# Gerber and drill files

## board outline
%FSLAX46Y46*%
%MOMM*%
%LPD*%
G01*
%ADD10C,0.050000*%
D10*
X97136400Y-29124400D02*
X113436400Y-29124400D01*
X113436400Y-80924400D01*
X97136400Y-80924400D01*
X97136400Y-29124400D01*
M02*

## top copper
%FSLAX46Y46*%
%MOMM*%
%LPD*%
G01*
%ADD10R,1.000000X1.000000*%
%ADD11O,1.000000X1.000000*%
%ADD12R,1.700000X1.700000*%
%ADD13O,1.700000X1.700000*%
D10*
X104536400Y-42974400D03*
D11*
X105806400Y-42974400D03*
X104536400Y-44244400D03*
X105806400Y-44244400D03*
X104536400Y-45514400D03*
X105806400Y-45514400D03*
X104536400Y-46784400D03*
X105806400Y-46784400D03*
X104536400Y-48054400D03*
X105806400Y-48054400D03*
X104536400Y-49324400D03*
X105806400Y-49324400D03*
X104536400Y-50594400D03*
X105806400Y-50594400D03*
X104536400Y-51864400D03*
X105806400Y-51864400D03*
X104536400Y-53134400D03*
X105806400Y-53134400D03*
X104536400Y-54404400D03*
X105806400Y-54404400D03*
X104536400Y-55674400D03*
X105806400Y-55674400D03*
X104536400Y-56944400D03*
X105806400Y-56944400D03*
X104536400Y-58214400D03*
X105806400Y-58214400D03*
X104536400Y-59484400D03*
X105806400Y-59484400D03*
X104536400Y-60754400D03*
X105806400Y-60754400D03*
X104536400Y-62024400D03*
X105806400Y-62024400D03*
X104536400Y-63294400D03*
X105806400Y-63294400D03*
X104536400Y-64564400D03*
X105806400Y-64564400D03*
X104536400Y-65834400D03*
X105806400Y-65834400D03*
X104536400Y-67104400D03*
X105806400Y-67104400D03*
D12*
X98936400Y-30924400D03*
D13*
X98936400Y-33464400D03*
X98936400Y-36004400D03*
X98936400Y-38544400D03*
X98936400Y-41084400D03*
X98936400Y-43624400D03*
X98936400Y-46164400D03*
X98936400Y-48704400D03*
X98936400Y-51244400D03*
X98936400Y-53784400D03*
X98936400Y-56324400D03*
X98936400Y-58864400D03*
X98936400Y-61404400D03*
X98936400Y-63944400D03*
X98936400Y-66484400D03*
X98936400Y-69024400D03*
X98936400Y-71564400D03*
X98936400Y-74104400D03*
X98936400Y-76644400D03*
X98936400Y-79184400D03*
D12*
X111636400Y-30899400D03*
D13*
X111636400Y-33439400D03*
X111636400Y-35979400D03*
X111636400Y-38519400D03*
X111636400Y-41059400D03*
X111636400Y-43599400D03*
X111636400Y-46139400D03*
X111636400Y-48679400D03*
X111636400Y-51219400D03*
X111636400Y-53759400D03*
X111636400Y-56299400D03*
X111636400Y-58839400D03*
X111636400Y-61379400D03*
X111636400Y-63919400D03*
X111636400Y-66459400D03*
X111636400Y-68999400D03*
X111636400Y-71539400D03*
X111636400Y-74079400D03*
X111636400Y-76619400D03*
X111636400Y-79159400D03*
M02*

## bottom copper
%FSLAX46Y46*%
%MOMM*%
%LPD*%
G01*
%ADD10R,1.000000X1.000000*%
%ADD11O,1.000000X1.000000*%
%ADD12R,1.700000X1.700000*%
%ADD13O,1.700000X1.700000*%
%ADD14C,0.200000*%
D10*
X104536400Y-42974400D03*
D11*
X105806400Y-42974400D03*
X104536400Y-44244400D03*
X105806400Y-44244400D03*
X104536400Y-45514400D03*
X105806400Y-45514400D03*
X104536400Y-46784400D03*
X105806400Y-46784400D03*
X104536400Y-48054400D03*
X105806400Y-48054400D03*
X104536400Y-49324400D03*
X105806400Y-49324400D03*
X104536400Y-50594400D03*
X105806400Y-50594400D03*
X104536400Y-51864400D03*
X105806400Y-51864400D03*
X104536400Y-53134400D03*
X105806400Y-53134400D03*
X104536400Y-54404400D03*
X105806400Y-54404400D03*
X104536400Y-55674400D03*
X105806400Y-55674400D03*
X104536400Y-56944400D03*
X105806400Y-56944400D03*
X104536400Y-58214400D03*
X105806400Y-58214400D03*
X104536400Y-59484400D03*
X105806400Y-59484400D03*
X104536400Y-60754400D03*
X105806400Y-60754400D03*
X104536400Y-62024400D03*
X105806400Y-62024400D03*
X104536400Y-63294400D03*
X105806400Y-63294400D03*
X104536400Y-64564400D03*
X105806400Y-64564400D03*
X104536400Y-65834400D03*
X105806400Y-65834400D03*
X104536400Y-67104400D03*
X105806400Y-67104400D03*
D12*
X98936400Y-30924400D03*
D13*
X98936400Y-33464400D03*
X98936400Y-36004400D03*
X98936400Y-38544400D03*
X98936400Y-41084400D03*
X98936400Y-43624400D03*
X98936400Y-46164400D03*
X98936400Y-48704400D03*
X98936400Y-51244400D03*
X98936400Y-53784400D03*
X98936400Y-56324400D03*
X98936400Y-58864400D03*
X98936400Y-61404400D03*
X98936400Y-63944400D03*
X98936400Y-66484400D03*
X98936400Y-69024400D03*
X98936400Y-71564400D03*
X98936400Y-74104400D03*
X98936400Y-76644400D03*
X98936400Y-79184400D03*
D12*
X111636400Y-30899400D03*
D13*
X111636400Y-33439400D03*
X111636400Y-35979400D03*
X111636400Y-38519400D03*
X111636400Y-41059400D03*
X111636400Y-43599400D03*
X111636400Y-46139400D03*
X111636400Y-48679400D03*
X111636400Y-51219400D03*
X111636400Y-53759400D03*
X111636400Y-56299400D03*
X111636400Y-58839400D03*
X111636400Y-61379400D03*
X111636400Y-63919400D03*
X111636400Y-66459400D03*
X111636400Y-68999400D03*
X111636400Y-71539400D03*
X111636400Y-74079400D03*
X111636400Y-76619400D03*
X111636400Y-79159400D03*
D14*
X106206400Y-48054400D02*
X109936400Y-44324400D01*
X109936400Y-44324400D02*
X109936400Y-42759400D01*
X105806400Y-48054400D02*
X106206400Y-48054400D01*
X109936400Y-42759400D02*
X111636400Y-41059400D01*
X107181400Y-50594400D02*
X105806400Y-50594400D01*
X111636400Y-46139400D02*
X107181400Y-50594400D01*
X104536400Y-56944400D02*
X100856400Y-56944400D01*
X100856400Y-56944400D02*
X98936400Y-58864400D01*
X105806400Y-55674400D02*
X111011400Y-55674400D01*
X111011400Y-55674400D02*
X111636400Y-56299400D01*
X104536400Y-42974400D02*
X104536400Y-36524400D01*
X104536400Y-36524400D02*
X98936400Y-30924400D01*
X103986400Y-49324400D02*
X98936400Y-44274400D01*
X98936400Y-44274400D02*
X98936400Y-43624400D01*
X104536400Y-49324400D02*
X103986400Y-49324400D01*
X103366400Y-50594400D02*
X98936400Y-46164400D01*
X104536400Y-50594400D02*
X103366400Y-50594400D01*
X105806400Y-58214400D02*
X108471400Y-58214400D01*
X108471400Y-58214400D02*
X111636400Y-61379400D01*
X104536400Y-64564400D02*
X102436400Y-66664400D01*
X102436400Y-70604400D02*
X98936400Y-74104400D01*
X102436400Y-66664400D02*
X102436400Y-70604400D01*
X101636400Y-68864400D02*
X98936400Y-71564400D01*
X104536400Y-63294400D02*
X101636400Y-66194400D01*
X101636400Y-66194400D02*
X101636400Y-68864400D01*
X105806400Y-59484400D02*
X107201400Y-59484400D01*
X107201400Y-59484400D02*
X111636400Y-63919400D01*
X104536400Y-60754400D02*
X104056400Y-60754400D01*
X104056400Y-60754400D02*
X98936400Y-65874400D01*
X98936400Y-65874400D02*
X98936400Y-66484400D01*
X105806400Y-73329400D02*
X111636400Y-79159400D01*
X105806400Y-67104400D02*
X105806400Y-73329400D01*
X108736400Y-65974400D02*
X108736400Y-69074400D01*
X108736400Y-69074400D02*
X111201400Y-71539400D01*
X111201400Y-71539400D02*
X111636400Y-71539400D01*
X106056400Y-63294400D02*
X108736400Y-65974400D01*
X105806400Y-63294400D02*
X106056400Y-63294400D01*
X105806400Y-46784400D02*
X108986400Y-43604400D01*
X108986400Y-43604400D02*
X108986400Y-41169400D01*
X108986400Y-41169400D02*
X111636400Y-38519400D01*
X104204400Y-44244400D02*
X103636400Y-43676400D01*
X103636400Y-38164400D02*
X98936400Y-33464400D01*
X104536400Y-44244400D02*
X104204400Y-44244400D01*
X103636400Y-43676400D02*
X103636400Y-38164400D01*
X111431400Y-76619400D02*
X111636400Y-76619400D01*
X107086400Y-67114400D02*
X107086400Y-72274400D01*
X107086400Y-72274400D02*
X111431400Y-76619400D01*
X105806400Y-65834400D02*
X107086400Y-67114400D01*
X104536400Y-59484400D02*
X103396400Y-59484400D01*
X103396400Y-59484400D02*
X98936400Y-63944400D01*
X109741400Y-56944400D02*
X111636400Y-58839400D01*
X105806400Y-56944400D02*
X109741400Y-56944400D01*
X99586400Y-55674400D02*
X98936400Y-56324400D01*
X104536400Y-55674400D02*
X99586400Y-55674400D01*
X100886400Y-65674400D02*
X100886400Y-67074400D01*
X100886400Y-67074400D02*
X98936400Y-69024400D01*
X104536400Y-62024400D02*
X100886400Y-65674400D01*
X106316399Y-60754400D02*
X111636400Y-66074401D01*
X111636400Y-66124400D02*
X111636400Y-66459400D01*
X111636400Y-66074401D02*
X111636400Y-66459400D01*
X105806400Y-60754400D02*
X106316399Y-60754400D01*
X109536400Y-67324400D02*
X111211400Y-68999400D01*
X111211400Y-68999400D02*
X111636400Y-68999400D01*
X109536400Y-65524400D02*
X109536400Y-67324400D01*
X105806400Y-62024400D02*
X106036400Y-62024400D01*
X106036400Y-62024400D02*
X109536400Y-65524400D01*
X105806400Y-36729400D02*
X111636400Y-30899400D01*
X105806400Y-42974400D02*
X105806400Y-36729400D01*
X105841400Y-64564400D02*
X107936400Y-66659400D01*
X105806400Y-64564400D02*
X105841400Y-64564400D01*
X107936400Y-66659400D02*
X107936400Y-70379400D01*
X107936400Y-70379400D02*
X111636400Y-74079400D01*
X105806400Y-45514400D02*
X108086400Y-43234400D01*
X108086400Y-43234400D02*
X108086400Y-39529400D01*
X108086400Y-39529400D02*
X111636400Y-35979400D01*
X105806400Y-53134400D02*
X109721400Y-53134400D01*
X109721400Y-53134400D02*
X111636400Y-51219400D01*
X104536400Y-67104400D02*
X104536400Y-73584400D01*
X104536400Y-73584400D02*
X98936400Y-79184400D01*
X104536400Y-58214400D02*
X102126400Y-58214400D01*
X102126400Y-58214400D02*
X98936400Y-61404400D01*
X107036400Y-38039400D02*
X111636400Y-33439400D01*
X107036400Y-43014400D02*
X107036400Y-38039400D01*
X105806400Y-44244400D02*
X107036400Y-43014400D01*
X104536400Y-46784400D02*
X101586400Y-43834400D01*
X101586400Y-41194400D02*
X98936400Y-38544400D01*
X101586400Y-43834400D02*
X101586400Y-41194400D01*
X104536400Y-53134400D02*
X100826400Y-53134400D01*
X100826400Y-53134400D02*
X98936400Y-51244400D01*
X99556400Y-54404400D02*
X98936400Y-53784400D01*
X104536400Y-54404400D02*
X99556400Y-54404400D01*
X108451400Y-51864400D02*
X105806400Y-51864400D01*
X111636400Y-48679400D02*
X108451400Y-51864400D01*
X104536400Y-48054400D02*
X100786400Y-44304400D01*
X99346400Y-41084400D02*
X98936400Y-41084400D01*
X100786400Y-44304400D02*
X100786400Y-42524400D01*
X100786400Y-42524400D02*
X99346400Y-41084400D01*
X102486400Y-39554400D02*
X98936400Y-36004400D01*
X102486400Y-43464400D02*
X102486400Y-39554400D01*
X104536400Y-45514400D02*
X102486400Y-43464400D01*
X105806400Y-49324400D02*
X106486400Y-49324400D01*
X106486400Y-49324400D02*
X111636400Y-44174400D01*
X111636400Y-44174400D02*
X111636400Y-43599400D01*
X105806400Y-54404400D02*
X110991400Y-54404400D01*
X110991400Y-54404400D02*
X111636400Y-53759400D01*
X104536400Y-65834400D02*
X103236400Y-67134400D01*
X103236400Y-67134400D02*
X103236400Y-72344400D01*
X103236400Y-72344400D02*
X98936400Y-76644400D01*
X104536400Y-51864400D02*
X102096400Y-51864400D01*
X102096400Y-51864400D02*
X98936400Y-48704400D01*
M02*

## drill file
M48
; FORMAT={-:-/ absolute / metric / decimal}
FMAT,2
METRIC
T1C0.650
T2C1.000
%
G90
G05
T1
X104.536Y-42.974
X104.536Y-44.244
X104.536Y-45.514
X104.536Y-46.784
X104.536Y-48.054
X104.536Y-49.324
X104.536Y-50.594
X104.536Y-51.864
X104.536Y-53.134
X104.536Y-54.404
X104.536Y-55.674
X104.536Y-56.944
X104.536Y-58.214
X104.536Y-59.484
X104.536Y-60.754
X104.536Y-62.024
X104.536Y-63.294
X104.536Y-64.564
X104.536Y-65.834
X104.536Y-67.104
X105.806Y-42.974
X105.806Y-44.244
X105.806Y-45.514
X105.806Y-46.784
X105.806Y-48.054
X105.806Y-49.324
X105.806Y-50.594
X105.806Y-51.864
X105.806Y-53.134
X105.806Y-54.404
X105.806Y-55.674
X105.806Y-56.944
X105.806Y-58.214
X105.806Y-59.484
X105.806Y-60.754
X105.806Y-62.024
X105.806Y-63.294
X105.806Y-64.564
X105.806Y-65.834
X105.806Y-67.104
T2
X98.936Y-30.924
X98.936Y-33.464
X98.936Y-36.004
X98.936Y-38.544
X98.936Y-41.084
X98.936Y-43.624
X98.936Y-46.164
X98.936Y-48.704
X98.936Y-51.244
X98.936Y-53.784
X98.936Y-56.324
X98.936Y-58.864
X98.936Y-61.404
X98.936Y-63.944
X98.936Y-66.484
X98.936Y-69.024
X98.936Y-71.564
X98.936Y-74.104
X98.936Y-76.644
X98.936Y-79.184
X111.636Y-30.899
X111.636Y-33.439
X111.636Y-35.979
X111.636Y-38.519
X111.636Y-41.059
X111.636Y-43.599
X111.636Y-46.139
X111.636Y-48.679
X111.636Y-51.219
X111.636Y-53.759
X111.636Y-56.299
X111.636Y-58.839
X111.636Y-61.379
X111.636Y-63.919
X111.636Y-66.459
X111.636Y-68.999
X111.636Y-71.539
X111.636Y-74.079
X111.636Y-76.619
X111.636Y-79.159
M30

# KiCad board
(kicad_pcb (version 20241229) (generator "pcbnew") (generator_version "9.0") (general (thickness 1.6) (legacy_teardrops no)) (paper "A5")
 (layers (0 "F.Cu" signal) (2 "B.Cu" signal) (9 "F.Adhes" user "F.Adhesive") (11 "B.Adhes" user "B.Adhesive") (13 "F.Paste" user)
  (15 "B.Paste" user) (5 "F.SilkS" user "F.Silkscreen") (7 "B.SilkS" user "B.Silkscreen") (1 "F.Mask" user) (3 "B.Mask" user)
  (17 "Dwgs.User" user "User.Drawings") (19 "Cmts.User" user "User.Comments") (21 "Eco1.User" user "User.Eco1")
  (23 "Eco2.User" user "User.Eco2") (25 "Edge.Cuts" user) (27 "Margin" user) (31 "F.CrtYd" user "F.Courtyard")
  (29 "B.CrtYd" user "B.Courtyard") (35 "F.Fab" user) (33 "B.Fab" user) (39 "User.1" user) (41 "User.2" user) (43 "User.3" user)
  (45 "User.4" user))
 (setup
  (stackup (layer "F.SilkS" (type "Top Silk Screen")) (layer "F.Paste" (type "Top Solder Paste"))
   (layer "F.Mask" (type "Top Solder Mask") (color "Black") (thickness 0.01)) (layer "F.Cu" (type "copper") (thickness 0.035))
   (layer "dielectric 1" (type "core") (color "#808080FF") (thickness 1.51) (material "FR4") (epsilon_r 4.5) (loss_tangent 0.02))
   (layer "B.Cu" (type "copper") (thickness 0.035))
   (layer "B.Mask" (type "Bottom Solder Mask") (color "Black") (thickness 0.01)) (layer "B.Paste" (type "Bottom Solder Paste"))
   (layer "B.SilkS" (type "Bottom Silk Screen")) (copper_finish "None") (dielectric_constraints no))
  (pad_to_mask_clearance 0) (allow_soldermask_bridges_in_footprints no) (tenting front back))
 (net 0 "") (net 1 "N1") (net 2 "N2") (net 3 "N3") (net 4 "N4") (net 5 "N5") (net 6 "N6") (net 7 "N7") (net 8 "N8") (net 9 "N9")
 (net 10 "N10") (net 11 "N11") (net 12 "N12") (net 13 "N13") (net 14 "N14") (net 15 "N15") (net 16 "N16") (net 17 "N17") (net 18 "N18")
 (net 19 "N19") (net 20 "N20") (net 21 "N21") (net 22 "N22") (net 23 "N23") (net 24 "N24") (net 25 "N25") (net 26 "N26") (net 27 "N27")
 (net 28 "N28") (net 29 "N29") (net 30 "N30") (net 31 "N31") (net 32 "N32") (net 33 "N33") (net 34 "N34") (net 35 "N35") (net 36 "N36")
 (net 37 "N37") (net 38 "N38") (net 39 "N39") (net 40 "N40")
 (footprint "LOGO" (layer "F.Cu") (at 105.3988 74.55 90)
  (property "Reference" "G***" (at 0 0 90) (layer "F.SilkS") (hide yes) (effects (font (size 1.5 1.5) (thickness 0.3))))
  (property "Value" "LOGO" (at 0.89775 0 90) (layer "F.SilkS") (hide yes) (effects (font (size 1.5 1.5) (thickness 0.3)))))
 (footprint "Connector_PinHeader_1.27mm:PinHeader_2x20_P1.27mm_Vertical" (layer "F.Cu") (at 104.5364 42.9744)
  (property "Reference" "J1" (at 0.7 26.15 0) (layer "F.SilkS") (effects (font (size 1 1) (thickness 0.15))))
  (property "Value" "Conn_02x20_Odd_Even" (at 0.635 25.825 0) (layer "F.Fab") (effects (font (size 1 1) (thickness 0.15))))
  (pad "1" thru_hole rect (at 0 0) (size 1 1) (drill 0.65) (layers "*.Cu" "*.Mask") (remove_unused_layers no) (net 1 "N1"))
  (pad "2" thru_hole oval (at 1.27 0) (size 1 1) (drill 0.65) (layers "*.Cu" "*.Mask") (remove_unused_layers no) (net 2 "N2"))
  (pad "3" thru_hole oval (at 0 1.27) (size 1 1) (drill 0.65) (layers "*.Cu" "*.Mask") (remove_unused_layers no) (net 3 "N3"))
  (pad "4" thru_hole oval (at 1.27 1.27) (size 1 1) (drill 0.65) (layers "*.Cu" "*.Mask") (remove_unused_layers no) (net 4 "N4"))
  (pad "5" thru_hole oval (at 0 2.54) (size 1 1) (drill 0.65) (layers "*.Cu" "*.Mask") (remove_unused_layers no) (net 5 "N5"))
  (pad "6" thru_hole oval (at 1.27 2.54) (size 1 1) (drill 0.65) (layers "*.Cu" "*.Mask") (remove_unused_layers no) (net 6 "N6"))
  (pad "7" thru_hole oval (at 0 3.81) (size 1 1) (drill 0.65) (layers "*.Cu" "*.Mask") (remove_unused_layers no) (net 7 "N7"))
  (pad "8" thru_hole oval (at 1.27 3.81) (size 1 1) (drill 0.65) (layers "*.Cu" "*.Mask") (remove_unused_layers no) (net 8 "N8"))
  (pad "9" thru_hole oval (at 0 5.08) (size 1 1) (drill 0.65) (layers "*.Cu" "*.Mask") (remove_unused_layers no) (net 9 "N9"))
  (pad "10" thru_hole oval (at 1.27 5.08) (size 1 1) (drill 0.65) (layers "*.Cu" "*.Mask") (remove_unused_layers no) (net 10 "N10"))
  (pad "11" thru_hole oval (at 0 6.35) (size 1 1) (drill 0.65) (layers "*.Cu" "*.Mask") (remove_unused_layers no) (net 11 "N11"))
  (pad "12" thru_hole oval (at 1.27 6.35) (size 1 1) (drill 0.65) (layers "*.Cu" "*.Mask") (remove_unused_layers no) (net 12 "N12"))
  (pad "13" thru_hole oval (at 0 7.62) (size 1 1) (drill 0.65) (layers "*.Cu" "*.Mask") (remove_unused_layers no) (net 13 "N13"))
  (pad "14" thru_hole oval (at 1.27 7.62) (size 1 1) (drill 0.65) (layers "*.Cu" "*.Mask") (remove_unused_layers no) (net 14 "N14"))
  (pad "15" thru_hole oval (at 0 8.89) (size 1 1) (drill 0.65) (layers "*.Cu" "*.Mask") (remove_unused_layers no) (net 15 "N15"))
  (pad "16" thru_hole oval (at 1.27 8.89) (size 1 1) (drill 0.65) (layers "*.Cu" "*.Mask") (remove_unused_layers no) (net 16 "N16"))
  (pad "17" thru_hole oval (at 0 10.16) (size 1 1) (drill 0.65) (layers "*.Cu" "*.Mask") (remove_unused_layers no) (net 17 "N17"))
  (pad "18" thru_hole oval (at 1.27 10.16) (size 1 1) (drill 0.65) (layers "*.Cu" "*.Mask") (remove_unused_layers no) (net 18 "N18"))
  (pad "19" thru_hole oval (at 0 11.43) (size 1 1) (drill 0.65) (layers "*.Cu" "*.Mask") (remove_unused_layers no) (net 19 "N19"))
  (pad "20" thru_hole oval (at 1.27 11.43) (size 1 1) (drill 0.65) (layers "*.Cu" "*.Mask") (remove_unused_layers no) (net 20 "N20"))
  (pad "21" thru_hole oval (at 0 12.7) (size 1 1) (drill 0.65) (layers "*.Cu" "*.Mask") (remove_unused_layers no) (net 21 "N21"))
  (pad "22" thru_hole oval (at 1.27 12.7) (size 1 1) (drill 0.65) (layers "*.Cu" "*.Mask") (remove_unused_layers no) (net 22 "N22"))
  (pad "23" thru_hole oval (at 0 13.97) (size 1 1) (drill 0.65) (layers "*.Cu" "*.Mask") (remove_unused_layers no) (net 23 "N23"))
  (pad "24" thru_hole oval (at 1.27 13.97) (size 1 1) (drill 0.65) (layers "*.Cu" "*.Mask") (remove_unused_layers no) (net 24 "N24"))
  (pad "25" thru_hole oval (at 0 15.24) (size 1 1) (drill 0.65) (layers "*.Cu" "*.Mask") (remove_unused_layers no) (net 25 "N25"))
  (pad "26" thru_hole oval (at 1.27 15.24) (size 1 1) (drill 0.65) (layers "*.Cu" "*.Mask") (remove_unused_layers no) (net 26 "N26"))
  (pad "27" thru_hole oval (at 0 16.51) (size 1 1) (drill 0.65) (layers "*.Cu" "*.Mask") (remove_unused_layers no) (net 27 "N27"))
  (pad "28" thru_hole oval (at 1.27 16.51) (size 1 1) (drill 0.65) (layers "*.Cu" "*.Mask") (remove_unused_layers no) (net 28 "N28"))
  (pad "29" thru_hole oval (at 0 17.78) (size 1 1) (drill 0.65) (layers "*.Cu" "*.Mask") (remove_unused_layers no) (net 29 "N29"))
  (pad "30" thru_hole oval (at 1.27 17.78) (size 1 1) (drill 0.65) (layers "*.Cu" "*.Mask") (remove_unused_layers no) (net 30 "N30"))
  (pad "31" thru_hole oval (at 0 19.05) (size 1 1) (drill 0.65) (layers "*.Cu" "*.Mask") (remove_unused_layers no) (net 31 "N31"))
  (pad "32" thru_hole oval (at 1.27 19.05) (size 1 1) (drill 0.65) (layers "*.Cu" "*.Mask") (remove_unused_layers no) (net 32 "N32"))
  (pad "33" thru_hole oval (at 0 20.32) (size 1 1) (drill 0.65) (layers "*.Cu" "*.Mask") (remove_unused_layers no) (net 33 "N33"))
  (pad "34" thru_hole oval (at 1.27 20.32) (size 1 1) (drill 0.65) (layers "*.Cu" "*.Mask") (remove_unused_layers no) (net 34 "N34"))
  (pad "35" thru_hole oval (at 0 21.59) (size 1 1) (drill 0.65) (layers "*.Cu" "*.Mask") (remove_unused_layers no) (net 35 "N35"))
  (pad "36" thru_hole oval (at 1.27 21.59) (size 1 1) (drill 0.65) (layers "*.Cu" "*.Mask") (remove_unused_layers no) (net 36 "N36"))
  (pad "37" thru_hole oval (at 0 22.86) (size 1 1) (drill 0.65) (layers "*.Cu" "*.Mask") (remove_unused_layers no) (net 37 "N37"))
  (pad "38" thru_hole oval (at 1.27 22.86) (size 1 1) (drill 0.65) (layers "*.Cu" "*.Mask") (remove_unused_layers no) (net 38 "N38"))
  (pad "39" thru_hole oval (at 0 24.13) (size 1 1) (drill 0.65) (layers "*.Cu" "*.Mask") (remove_unused_layers no) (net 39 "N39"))
  (pad "40" thru_hole oval (at 1.27 24.13) (size 1 1) (drill 0.65) (layers "*.Cu" "*.Mask") (remove_unused_layers no) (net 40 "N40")))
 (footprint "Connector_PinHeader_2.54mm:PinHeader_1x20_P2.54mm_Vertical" (layer "B.Cu") (at 98.9364 30.9244 180)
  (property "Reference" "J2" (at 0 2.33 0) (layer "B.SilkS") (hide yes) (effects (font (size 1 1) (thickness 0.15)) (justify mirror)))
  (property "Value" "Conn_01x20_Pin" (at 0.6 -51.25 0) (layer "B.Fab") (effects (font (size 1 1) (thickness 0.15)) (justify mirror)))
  (pad "1" thru_hole rect (at 0 0 180) (size 1.7 1.7) (drill 1) (layers "*.Cu" "*.Mask") (remove_unused_layers no) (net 1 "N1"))
  (pad "2" thru_hole oval (at 0 -2.54 180) (size 1.7 1.7) (drill 1) (layers "*.Cu" "*.Mask") (remove_unused_layers no) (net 3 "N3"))
  (pad "3" thru_hole oval (at 0 -5.08 180) (size 1.7 1.7) (drill 1) (layers "*.Cu" "*.Mask") (remove_unused_layers no) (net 5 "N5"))
  (pad "4" thru_hole oval (at 0 -7.62 180) (size 1.7 1.7) (drill 1) (layers "*.Cu" "*.Mask") (remove_unused_layers no) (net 7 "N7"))
  (pad "5" thru_hole oval (at 0 -10.16 180) (size 1.7 1.7) (drill 1) (layers "*.Cu" "*.Mask") (remove_unused_layers no) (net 9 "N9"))
  (pad "6" thru_hole oval (at 0 -12.7 180) (size 1.7 1.7) (drill 1) (layers "*.Cu" "*.Mask") (remove_unused_layers no) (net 11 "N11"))
  (pad "7" thru_hole oval (at 0 -15.24 180) (size 1.7 1.7) (drill 1) (layers "*.Cu" "*.Mask") (remove_unused_layers no) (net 13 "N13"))
  (pad "8" thru_hole oval (at 0 -17.78 180) (size 1.7 1.7) (drill 1) (layers "*.Cu" "*.Mask") (remove_unused_layers no) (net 15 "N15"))
  (pad "9" thru_hole oval (at 0 -20.32 180) (size 1.7 1.7) (drill 1) (layers "*.Cu" "*.Mask") (remove_unused_layers no) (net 17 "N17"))
  (pad "10" thru_hole oval (at 0 -22.86 180) (size 1.7 1.7) (drill 1) (layers "*.Cu" "*.Mask") (remove_unused_layers no) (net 19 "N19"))
  (pad "11" thru_hole oval (at 0 -25.4 180) (size 1.7 1.7) (drill 1) (layers "*.Cu" "*.Mask") (remove_unused_layers no) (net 21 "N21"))
  (pad "12" thru_hole oval (at 0 -27.94 180) (size 1.7 1.7) (drill 1) (layers "*.Cu" "*.Mask") (remove_unused_layers no) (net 23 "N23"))
  (pad "13" thru_hole oval (at 0 -30.48 180) (size 1.7 1.7) (drill 1) (layers "*.Cu" "*.Mask") (remove_unused_layers no) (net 25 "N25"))
  (pad "14" thru_hole oval (at 0 -33.02 180) (size 1.7 1.7) (drill 1) (layers "*.Cu" "*.Mask") (remove_unused_layers no) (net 27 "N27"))
  (pad "15" thru_hole oval (at 0 -35.56 180) (size 1.7 1.7) (drill 1) (layers "*.Cu" "*.Mask") (remove_unused_layers no) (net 29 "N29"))
  (pad "16" thru_hole oval (at 0 -38.1 180) (size 1.7 1.7) (drill 1) (layers "*.Cu" "*.Mask") (remove_unused_layers no) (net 31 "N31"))
  (pad "17" thru_hole oval (at 0 -40.64 180) (size 1.7 1.7) (drill 1) (layers "*.Cu" "*.Mask") (remove_unused_layers no) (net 33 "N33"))
  (pad "18" thru_hole oval (at 0 -43.18 180) (size 1.7 1.7) (drill 1) (layers "*.Cu" "*.Mask") (remove_unused_layers no) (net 35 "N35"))
  (pad "19" thru_hole oval (at 0 -45.72 180) (size 1.7 1.7) (drill 1) (layers "*.Cu" "*.Mask") (remove_unused_layers no) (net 37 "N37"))
  (pad "20" thru_hole oval (at 0 -48.26 180) (size 1.7 1.7) (drill 1) (layers "*.Cu" "*.Mask") (remove_unused_layers no) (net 39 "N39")))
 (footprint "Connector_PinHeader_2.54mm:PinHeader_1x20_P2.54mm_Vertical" (layer "B.Cu") (at 111.6364 30.8994 180)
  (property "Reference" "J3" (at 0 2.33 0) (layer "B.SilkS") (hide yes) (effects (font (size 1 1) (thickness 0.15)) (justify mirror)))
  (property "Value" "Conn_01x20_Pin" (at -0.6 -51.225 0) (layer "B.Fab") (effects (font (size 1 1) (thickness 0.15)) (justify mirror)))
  (pad "1" thru_hole rect (at 0 0 180) (size 1.7 1.7) (drill 1) (layers "*.Cu" "*.Mask") (remove_unused_layers no) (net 2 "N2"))
  (pad "2" thru_hole oval (at 0 -2.54 180) (size 1.7 1.7) (drill 1) (layers "*.Cu" "*.Mask") (remove_unused_layers no) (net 4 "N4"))
  (pad "3" thru_hole oval (at 0 -5.08 180) (size 1.7 1.7) (drill 1) (layers "*.Cu" "*.Mask") (remove_unused_layers no) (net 6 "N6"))
  (pad "4" thru_hole oval (at 0 -7.62 180) (size 1.7 1.7) (drill 1) (layers "*.Cu" "*.Mask") (remove_unused_layers no) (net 8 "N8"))
  (pad "5" thru_hole oval (at 0 -10.16 180) (size 1.7 1.7) (drill 1) (layers "*.Cu" "*.Mask") (remove_unused_layers no) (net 10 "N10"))
  (pad "6" thru_hole oval (at 0 -12.7 180) (size 1.7 1.7) (drill 1) (layers "*.Cu" "*.Mask") (remove_unused_layers no) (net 12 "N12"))
  (pad "7" thru_hole oval (at 0 -15.24 180) (size 1.7 1.7) (drill 1) (layers "*.Cu" "*.Mask") (remove_unused_layers no) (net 14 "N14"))
  (pad "8" thru_hole oval (at 0 -17.78 180) (size 1.7 1.7) (drill 1) (layers "*.Cu" "*.Mask") (remove_unused_layers no) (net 16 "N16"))
  (pad "9" thru_hole oval (at 0 -20.32 180) (size 1.7 1.7) (drill 1) (layers "*.Cu" "*.Mask") (remove_unused_layers no) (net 18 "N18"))
  (pad "10" thru_hole oval (at 0 -22.86 180) (size 1.7 1.7) (drill 1) (layers "*.Cu" "*.Mask") (remove_unused_layers no) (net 20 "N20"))
  (pad "11" thru_hole oval (at 0 -25.4 180) (size 1.7 1.7) (drill 1) (layers "*.Cu" "*.Mask") (remove_unused_layers no) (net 22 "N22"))
  (pad "12" thru_hole oval (at 0 -27.94 180) (size 1.7 1.7) (drill 1) (layers "*.Cu" "*.Mask") (remove_unused_layers no) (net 24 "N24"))
  (pad "13" thru_hole oval (at 0 -30.48 180) (size 1.7 1.7) (drill 1) (layers "*.Cu" "*.Mask") (remove_unused_layers no) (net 26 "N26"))
  (pad "14" thru_hole oval (at 0 -33.02 180) (size 1.7 1.7) (drill 1) (layers "*.Cu" "*.Mask") (remove_unused_layers no) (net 28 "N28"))
  (pad "15" thru_hole oval (at 0 -35.56 180) (size 1.7 1.7) (drill 1) (layers "*.Cu" "*.Mask") (remove_unused_layers no) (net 30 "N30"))
  (pad "16" thru_hole oval (at 0 -38.1 180) (size 1.7 1.7) (drill 1) (layers "*.Cu" "*.Mask") (remove_unused_layers no) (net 32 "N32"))
  (pad "17" thru_hole oval (at 0 -40.64 180) (size 1.7 1.7) (drill 1) (layers "*.Cu" "*.Mask") (remove_unused_layers no) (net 34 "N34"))
  (pad "18" thru_hole oval (at 0 -43.18 180) (size 1.7 1.7) (drill 1) (layers "*.Cu" "*.Mask") (remove_unused_layers no) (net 36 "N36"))
  (pad "19" thru_hole oval (at 0 -45.72 180) (size 1.7 1.7) (drill 1) (layers "*.Cu" "*.Mask") (remove_unused_layers no) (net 38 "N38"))
  (pad "20" thru_hole oval (at 0 -48.26 180) (size 1.7 1.7) (drill 1) (layers "*.Cu" "*.Mask") (remove_unused_layers no) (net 40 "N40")))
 (gr_rect (start 97.1364 29.1244) (end 113.4364 80.9244) (stroke (width 0.05) (type default)) (fill no) (layer "Edge.Cuts"))
 (segment (start 106.2064 48.0544) (end 109.9364 44.3244) (width 0.2) (layer "B.Cu") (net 10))
 (segment (start 109.9364 44.3244) (end 109.9364 42.7594) (width 0.2) (layer "B.Cu") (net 10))
 (segment (start 105.8064 48.0544) (end 106.2064 48.0544) (width 0.2) (layer "B.Cu") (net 10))
 (segment (start 109.9364 42.7594) (end 111.6364 41.0594) (width 0.2) (layer "B.Cu") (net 10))
 (segment (start 107.1814 50.5944) (end 105.8064 50.5944) (width 0.2) (layer "B.Cu") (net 14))
 (segment (start 111.6364 46.1394) (end 107.1814 50.5944) (width 0.2) (layer "B.Cu") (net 14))
 (segment (start 104.5364 56.9444) (end 100.8564 56.9444) (width 0.2) (layer "B.Cu") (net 23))
 (segment (start 100.8564 56.9444) (end 98.9364 58.8644) (width 0.2) (layer "B.Cu") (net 23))
 (segment (start 105.8064 55.6744) (end 111.0114 55.6744) (width 0.2) (layer "B.Cu") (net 22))
 (segment (start 111.0114 55.6744) (end 111.6364 56.2994) (width 0.2) (layer "B.Cu") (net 22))
 (segment (start 104.5364 42.9744) (end 104.5364 36.5244) (width 0.2) (layer "B.Cu") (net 1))
 (segment (start 104.5364 36.5244) (end 98.9364 30.9244) (width 0.2) (layer "B.Cu") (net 1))
 (segment (start 103.9864 49.3244) (end 98.9364 44.2744) (width 0.2) (layer "B.Cu") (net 11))
 (segment (start 98.9364 44.2744) (end 98.9364 43.6244) (width 0.2) (layer "B.Cu") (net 11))
 (segment (start 104.5364 49.3244) (end 103.9864 49.3244) (width 0.2) (layer "B.Cu") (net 11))
 (segment (start 103.3664 50.5944) (end 98.9364 46.1644) (width 0.2) (layer "B.Cu") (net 13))
 (segment (start 104.5364 50.5944) (end 103.3664 50.5944) (width 0.2) (layer "B.Cu") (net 13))
 (segment (start 105.8064 58.2144) (end 108.4714 58.2144) (width 0.2) (layer "B.Cu") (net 26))
 (segment (start 108.4714 58.2144) (end 111.6364 61.3794) (width 0.2) (layer "B.Cu") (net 26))
 (segment (start 104.5364 64.5644) (end 102.4364 66.6644) (width 0.2) (layer "B.Cu") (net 35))
 (segment (start 102.4364 70.6044) (end 98.9364 74.1044) (width 0.2) (layer "B.Cu") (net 35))
 (segment (start 102.4364 66.6644) (end 102.4364 70.6044) (width 0.2) (layer "B.Cu") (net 35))
 (segment (start 101.6364 68.8644) (end 98.9364 71.5644) (width 0.2) (layer "B.Cu") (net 33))
 (segment (start 104.5364 63.2944) (end 101.6364 66.1944) (width 0.2) (layer "B.Cu") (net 33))
 (segment (start 101.6364 66.1944) (end 101.6364 68.8644) (width 0.2) (layer "B.Cu") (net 33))
 (segment (start 105.8064 59.4844) (end 107.2014 59.4844) (width 0.2) (layer "B.Cu") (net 28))
 (segment (start 107.2014 59.4844) (end 111.6364 63.9194) (width 0.2) (layer "B.Cu") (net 28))
 (segment (start 104.5364 60.7544) (end 104.0564 60.7544) (width 0.2) (layer "B.Cu") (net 29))
 (segment (start 104.0564 60.7544) (end 98.9364 65.8744) (width 0.2) (layer "B.Cu") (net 29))
 (segment (start 98.9364 65.8744) (end 98.9364 66.4844) (width 0.2) (layer "B.Cu") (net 29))
 (segment (start 105.8064 73.3294) (end 111.6364 79.1594) (width 0.2) (layer "B.Cu") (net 40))
 (segment (start 105.8064 67.1044) (end 105.8064 73.3294) (width 0.2) (layer "B.Cu") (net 40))
 (segment (start 108.7364 65.9744) (end 108.7364 69.0744) (width 0.2) (layer "B.Cu") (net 34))
 (segment (start 108.7364 69.0744) (end 111.2014 71.5394) (width 0.2) (layer "B.Cu") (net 34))
 (segment (start 111.2014 71.5394) (end 111.6364 71.5394) (width 0.2) (layer "B.Cu") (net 34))
 (segment (start 106.0564 63.2944) (end 108.7364 65.9744) (width 0.2) (layer "B.Cu") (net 34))
 (segment (start 105.8064 63.2944) (end 106.0564 63.2944) (width 0.2) (layer "B.Cu") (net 34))
 (segment (start 105.8064 46.7844) (end 108.9864 43.6044) (width 0.2) (layer "B.Cu") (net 8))
 (segment (start 108.9864 43.6044) (end 108.9864 41.1694) (width 0.2) (layer "B.Cu") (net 8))
 (segment (start 108.9864 41.1694) (end 111.6364 38.5194) (width 0.2) (layer "B.Cu") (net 8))
 (segment (start 104.2044 44.2444) (end 103.6364 43.6764) (width 0.2) (layer "B.Cu") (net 3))
 (segment (start 103.6364 38.1644) (end 98.9364 33.4644) (width 0.2) (layer "B.Cu") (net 3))
 (segment (start 104.5364 44.2444) (end 104.2044 44.2444) (width 0.2) (layer "B.Cu") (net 3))
 (segment (start 103.6364 43.6764) (end 103.6364 38.1644) (width 0.2) (layer "B.Cu") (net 3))
 (segment (start 111.4314 76.6194) (end 111.6364 76.6194) (width 0.2) (layer "B.Cu") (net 38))
 (segment (start 107.0864 67.1144) (end 107.0864 72.2744) (width 0.2) (layer "B.Cu") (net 38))
 (segment (start 107.0864 72.2744) (end 111.4314 76.6194) (width 0.2) (layer "B.Cu") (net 38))
 (segment (start 105.8064 65.8344) (end 107.0864 67.1144) (width 0.2) (layer "B.Cu") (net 38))
 (segment (start 104.5364 59.4844) (end 103.3964 59.4844) (width 0.2) (layer "B.Cu") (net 27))
 (segment (start 103.3964 59.4844) (end 98.9364 63.9444) (width 0.2) (layer "B.Cu") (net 27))
 (segment (start 109.7414 56.9444) (end 111.6364 58.8394) (width 0.2) (layer "B.Cu") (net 24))
 (segment (start 105.8064 56.9444) (end 109.7414 56.9444) (width 0.2) (layer "B.Cu") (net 24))
 (segment (start 99.5864 55.6744) (end 98.9364 56.3244) (width 0.2) (layer "B.Cu") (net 21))
 (segment (start 104.5364 55.6744) (end 99.5864 55.6744) (width 0.2) (layer "B.Cu") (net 21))
 (segment (start 100.8864 65.6744) (end 100.8864 67.0744) (width 0.2) (layer "B.Cu") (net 31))
 (segment (start 100.8864 67.0744) (end 98.9364 69.0244) (width 0.2) (layer "B.Cu") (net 31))
 (segment (start 104.5364 62.0244) (end 100.8864 65.6744) (width 0.2) (layer "B.Cu") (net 31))
 (segment (start 106.316399 60.7544) (end 111.6364 66.074401) (width 0.2) (layer "B.Cu") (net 30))
 (segment (start 111.6364 66.1244) (end 111.6364 66.4594) (width 0.2) (layer "B.Cu") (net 30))
 (segment (start 111.6364 66.074401) (end 111.6364 66.4594) (width 0.2) (layer "B.Cu") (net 30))
 (segment (start 105.8064 60.7544) (end 106.316399 60.7544) (width 0.2) (layer "B.Cu") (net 30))
 (segment (start 109.5364 67.3244) (end 111.2114 68.9994) (width 0.2) (layer "B.Cu") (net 32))
 (segment (start 111.2114 68.9994) (end 111.6364 68.9994) (width 0.2) (layer "B.Cu") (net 32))
 (segment (start 109.5364 65.5244) (end 109.5364 67.3244) (width 0.2) (layer "B.Cu") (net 32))
 (segment (start 105.8064 62.0244) (end 106.0364 62.0244) (width 0.2) (layer "B.Cu") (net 32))
 (segment (start 106.0364 62.0244) (end 109.5364 65.5244) (width 0.2) (layer "B.Cu") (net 32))
 (segment (start 105.8064 36.7294) (end 111.6364 30.8994) (width 0.2) (layer "B.Cu") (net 2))
 (segment (start 105.8064 42.9744) (end 105.8064 36.7294) (width 0.2) (layer "B.Cu") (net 2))
 (segment (start 105.8414 64.5644) (end 107.9364 66.6594) (width 0.2) (layer "B.Cu") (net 36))
 (segment (start 105.8064 64.5644) (end 105.8414 64.5644) (width 0.2) (layer "B.Cu") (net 36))
 (segment (start 107.9364 66.6594) (end 107.9364 70.3794) (width 0.2) (layer "B.Cu") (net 36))
 (segment (start 107.9364 70.3794) (end 111.6364 74.0794) (width 0.2) (layer "B.Cu") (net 36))
 (segment (start 105.8064 45.5144) (end 108.0864 43.2344) (width 0.2) (layer "B.Cu") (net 6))
 (segment (start 108.0864 43.2344) (end 108.0864 39.5294) (width 0.2) (layer "B.Cu") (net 6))
 (segment (start 108.0864 39.5294) (end 111.6364 35.9794) (width 0.2) (layer "B.Cu") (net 6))
 (segment (start 105.8064 53.1344) (end 109.7214 53.1344) (width 0.2) (layer "B.Cu") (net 18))
 (segment (start 109.7214 53.1344) (end 111.6364 51.2194) (width 0.2) (layer "B.Cu") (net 18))
 (segment (start 104.5364 67.1044) (end 104.5364 73.5844) (width 0.2) (layer "B.Cu") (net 39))
 (segment (start 104.5364 73.5844) (end 98.9364 79.1844) (width 0.2) (layer "B.Cu") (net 39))
 (segment (start 104.5364 58.2144) (end 102.1264 58.2144) (width 0.2) (layer "B.Cu") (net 25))
 (segment (start 102.1264 58.2144) (end 98.9364 61.4044) (width 0.2) (layer "B.Cu") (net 25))
 (segment (start 107.0364 38.0394) (end 111.6364 33.4394) (width 0.2) (layer "B.Cu") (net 4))
 (segment (start 107.0364 43.0144) (end 107.0364 38.0394) (width 0.2) (layer "B.Cu") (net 4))
 (segment (start 105.8064 44.2444) (end 107.0364 43.0144) (width 0.2) (layer "B.Cu") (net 4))
 (segment (start 104.5364 46.7844) (end 101.5864 43.8344) (width 0.2) (layer "B.Cu") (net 7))
 (segment (start 101.5864 41.1944) (end 98.9364 38.5444) (width 0.2) (layer "B.Cu") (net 7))
 (segment (start 101.5864 43.8344) (end 101.5864 41.1944) (width 0.2) (layer "B.Cu") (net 7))
 (segment (start 104.5364 53.1344) (end 100.8264 53.1344) (width 0.2) (layer "B.Cu") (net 17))
 (segment (start 100.8264 53.1344) (end 98.9364 51.2444) (width 0.2) (layer "B.Cu") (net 17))
 (segment (start 99.5564 54.4044) (end 98.9364 53.7844) (width 0.2) (layer "B.Cu") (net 19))
 (segment (start 104.5364 54.4044) (end 99.5564 54.4044) (width 0.2) (layer "B.Cu") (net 19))
 (segment (start 108.4514 51.8644) (end 105.8064 51.8644) (width 0.2) (layer "B.Cu") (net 16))
 (segment (start 111.6364 48.6794) (end 108.4514 51.8644) (width 0.2) (layer "B.Cu") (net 16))
 (segment (start 104.5364 48.0544) (end 100.7864 44.3044) (width 0.2) (layer "B.Cu") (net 9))
 (segment (start 99.3464 41.0844) (end 98.9364 41.0844) (width 0.2) (layer "B.Cu") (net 9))
 (segment (start 100.7864 44.3044) (end 100.7864 42.5244) (width 0.2) (layer "B.Cu") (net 9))
 (segment (start 100.7864 42.5244) (end 99.3464 41.0844) (width 0.2) (layer "B.Cu") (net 9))
 (segment (start 102.4864 39.5544) (end 98.9364 36.0044) (width 0.2) (layer "B.Cu") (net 5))
 (segment (start 102.4864 43.4644) (end 102.4864 39.5544) (width 0.2) (layer "B.Cu") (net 5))
 (segment (start 104.5364 45.5144) (end 102.4864 43.4644) (width 0.2) (layer "B.Cu") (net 5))
 (segment (start 105.8064 49.3244) (end 106.4864 49.3244) (width 0.2) (layer "B.Cu") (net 12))
 (segment (start 106.4864 49.3244) (end 111.6364 44.1744) (width 0.2) (layer "B.Cu") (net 12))
 (segment (start 111.6364 44.1744) (end 111.6364 43.5994) (width 0.2) (layer "B.Cu") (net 12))
 (segment (start 105.8064 54.4044) (end 110.9914 54.4044) (width 0.2) (layer "B.Cu") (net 20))
 (segment (start 110.9914 54.4044) (end 111.6364 53.7594) (width 0.2) (layer "B.Cu") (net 20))
 (segment (start 104.5364 65.8344) (end 103.2364 67.1344) (width 0.2) (layer "B.Cu") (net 37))
 (segment (start 103.2364 67.1344) (end 103.2364 72.3444) (width 0.2) (layer "B.Cu") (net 37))
 (segment (start 103.2364 72.3444) (end 98.9364 76.6444) (width 0.2) (layer "B.Cu") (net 37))
 (segment (start 104.5364 51.8644) (end 102.0964 51.8644) (width 0.2) (layer "B.Cu") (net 15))
 (segment (start 102.0964 51.8644) (end 98.9364 48.7044) (width 0.2) (layer "B.Cu") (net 15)))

